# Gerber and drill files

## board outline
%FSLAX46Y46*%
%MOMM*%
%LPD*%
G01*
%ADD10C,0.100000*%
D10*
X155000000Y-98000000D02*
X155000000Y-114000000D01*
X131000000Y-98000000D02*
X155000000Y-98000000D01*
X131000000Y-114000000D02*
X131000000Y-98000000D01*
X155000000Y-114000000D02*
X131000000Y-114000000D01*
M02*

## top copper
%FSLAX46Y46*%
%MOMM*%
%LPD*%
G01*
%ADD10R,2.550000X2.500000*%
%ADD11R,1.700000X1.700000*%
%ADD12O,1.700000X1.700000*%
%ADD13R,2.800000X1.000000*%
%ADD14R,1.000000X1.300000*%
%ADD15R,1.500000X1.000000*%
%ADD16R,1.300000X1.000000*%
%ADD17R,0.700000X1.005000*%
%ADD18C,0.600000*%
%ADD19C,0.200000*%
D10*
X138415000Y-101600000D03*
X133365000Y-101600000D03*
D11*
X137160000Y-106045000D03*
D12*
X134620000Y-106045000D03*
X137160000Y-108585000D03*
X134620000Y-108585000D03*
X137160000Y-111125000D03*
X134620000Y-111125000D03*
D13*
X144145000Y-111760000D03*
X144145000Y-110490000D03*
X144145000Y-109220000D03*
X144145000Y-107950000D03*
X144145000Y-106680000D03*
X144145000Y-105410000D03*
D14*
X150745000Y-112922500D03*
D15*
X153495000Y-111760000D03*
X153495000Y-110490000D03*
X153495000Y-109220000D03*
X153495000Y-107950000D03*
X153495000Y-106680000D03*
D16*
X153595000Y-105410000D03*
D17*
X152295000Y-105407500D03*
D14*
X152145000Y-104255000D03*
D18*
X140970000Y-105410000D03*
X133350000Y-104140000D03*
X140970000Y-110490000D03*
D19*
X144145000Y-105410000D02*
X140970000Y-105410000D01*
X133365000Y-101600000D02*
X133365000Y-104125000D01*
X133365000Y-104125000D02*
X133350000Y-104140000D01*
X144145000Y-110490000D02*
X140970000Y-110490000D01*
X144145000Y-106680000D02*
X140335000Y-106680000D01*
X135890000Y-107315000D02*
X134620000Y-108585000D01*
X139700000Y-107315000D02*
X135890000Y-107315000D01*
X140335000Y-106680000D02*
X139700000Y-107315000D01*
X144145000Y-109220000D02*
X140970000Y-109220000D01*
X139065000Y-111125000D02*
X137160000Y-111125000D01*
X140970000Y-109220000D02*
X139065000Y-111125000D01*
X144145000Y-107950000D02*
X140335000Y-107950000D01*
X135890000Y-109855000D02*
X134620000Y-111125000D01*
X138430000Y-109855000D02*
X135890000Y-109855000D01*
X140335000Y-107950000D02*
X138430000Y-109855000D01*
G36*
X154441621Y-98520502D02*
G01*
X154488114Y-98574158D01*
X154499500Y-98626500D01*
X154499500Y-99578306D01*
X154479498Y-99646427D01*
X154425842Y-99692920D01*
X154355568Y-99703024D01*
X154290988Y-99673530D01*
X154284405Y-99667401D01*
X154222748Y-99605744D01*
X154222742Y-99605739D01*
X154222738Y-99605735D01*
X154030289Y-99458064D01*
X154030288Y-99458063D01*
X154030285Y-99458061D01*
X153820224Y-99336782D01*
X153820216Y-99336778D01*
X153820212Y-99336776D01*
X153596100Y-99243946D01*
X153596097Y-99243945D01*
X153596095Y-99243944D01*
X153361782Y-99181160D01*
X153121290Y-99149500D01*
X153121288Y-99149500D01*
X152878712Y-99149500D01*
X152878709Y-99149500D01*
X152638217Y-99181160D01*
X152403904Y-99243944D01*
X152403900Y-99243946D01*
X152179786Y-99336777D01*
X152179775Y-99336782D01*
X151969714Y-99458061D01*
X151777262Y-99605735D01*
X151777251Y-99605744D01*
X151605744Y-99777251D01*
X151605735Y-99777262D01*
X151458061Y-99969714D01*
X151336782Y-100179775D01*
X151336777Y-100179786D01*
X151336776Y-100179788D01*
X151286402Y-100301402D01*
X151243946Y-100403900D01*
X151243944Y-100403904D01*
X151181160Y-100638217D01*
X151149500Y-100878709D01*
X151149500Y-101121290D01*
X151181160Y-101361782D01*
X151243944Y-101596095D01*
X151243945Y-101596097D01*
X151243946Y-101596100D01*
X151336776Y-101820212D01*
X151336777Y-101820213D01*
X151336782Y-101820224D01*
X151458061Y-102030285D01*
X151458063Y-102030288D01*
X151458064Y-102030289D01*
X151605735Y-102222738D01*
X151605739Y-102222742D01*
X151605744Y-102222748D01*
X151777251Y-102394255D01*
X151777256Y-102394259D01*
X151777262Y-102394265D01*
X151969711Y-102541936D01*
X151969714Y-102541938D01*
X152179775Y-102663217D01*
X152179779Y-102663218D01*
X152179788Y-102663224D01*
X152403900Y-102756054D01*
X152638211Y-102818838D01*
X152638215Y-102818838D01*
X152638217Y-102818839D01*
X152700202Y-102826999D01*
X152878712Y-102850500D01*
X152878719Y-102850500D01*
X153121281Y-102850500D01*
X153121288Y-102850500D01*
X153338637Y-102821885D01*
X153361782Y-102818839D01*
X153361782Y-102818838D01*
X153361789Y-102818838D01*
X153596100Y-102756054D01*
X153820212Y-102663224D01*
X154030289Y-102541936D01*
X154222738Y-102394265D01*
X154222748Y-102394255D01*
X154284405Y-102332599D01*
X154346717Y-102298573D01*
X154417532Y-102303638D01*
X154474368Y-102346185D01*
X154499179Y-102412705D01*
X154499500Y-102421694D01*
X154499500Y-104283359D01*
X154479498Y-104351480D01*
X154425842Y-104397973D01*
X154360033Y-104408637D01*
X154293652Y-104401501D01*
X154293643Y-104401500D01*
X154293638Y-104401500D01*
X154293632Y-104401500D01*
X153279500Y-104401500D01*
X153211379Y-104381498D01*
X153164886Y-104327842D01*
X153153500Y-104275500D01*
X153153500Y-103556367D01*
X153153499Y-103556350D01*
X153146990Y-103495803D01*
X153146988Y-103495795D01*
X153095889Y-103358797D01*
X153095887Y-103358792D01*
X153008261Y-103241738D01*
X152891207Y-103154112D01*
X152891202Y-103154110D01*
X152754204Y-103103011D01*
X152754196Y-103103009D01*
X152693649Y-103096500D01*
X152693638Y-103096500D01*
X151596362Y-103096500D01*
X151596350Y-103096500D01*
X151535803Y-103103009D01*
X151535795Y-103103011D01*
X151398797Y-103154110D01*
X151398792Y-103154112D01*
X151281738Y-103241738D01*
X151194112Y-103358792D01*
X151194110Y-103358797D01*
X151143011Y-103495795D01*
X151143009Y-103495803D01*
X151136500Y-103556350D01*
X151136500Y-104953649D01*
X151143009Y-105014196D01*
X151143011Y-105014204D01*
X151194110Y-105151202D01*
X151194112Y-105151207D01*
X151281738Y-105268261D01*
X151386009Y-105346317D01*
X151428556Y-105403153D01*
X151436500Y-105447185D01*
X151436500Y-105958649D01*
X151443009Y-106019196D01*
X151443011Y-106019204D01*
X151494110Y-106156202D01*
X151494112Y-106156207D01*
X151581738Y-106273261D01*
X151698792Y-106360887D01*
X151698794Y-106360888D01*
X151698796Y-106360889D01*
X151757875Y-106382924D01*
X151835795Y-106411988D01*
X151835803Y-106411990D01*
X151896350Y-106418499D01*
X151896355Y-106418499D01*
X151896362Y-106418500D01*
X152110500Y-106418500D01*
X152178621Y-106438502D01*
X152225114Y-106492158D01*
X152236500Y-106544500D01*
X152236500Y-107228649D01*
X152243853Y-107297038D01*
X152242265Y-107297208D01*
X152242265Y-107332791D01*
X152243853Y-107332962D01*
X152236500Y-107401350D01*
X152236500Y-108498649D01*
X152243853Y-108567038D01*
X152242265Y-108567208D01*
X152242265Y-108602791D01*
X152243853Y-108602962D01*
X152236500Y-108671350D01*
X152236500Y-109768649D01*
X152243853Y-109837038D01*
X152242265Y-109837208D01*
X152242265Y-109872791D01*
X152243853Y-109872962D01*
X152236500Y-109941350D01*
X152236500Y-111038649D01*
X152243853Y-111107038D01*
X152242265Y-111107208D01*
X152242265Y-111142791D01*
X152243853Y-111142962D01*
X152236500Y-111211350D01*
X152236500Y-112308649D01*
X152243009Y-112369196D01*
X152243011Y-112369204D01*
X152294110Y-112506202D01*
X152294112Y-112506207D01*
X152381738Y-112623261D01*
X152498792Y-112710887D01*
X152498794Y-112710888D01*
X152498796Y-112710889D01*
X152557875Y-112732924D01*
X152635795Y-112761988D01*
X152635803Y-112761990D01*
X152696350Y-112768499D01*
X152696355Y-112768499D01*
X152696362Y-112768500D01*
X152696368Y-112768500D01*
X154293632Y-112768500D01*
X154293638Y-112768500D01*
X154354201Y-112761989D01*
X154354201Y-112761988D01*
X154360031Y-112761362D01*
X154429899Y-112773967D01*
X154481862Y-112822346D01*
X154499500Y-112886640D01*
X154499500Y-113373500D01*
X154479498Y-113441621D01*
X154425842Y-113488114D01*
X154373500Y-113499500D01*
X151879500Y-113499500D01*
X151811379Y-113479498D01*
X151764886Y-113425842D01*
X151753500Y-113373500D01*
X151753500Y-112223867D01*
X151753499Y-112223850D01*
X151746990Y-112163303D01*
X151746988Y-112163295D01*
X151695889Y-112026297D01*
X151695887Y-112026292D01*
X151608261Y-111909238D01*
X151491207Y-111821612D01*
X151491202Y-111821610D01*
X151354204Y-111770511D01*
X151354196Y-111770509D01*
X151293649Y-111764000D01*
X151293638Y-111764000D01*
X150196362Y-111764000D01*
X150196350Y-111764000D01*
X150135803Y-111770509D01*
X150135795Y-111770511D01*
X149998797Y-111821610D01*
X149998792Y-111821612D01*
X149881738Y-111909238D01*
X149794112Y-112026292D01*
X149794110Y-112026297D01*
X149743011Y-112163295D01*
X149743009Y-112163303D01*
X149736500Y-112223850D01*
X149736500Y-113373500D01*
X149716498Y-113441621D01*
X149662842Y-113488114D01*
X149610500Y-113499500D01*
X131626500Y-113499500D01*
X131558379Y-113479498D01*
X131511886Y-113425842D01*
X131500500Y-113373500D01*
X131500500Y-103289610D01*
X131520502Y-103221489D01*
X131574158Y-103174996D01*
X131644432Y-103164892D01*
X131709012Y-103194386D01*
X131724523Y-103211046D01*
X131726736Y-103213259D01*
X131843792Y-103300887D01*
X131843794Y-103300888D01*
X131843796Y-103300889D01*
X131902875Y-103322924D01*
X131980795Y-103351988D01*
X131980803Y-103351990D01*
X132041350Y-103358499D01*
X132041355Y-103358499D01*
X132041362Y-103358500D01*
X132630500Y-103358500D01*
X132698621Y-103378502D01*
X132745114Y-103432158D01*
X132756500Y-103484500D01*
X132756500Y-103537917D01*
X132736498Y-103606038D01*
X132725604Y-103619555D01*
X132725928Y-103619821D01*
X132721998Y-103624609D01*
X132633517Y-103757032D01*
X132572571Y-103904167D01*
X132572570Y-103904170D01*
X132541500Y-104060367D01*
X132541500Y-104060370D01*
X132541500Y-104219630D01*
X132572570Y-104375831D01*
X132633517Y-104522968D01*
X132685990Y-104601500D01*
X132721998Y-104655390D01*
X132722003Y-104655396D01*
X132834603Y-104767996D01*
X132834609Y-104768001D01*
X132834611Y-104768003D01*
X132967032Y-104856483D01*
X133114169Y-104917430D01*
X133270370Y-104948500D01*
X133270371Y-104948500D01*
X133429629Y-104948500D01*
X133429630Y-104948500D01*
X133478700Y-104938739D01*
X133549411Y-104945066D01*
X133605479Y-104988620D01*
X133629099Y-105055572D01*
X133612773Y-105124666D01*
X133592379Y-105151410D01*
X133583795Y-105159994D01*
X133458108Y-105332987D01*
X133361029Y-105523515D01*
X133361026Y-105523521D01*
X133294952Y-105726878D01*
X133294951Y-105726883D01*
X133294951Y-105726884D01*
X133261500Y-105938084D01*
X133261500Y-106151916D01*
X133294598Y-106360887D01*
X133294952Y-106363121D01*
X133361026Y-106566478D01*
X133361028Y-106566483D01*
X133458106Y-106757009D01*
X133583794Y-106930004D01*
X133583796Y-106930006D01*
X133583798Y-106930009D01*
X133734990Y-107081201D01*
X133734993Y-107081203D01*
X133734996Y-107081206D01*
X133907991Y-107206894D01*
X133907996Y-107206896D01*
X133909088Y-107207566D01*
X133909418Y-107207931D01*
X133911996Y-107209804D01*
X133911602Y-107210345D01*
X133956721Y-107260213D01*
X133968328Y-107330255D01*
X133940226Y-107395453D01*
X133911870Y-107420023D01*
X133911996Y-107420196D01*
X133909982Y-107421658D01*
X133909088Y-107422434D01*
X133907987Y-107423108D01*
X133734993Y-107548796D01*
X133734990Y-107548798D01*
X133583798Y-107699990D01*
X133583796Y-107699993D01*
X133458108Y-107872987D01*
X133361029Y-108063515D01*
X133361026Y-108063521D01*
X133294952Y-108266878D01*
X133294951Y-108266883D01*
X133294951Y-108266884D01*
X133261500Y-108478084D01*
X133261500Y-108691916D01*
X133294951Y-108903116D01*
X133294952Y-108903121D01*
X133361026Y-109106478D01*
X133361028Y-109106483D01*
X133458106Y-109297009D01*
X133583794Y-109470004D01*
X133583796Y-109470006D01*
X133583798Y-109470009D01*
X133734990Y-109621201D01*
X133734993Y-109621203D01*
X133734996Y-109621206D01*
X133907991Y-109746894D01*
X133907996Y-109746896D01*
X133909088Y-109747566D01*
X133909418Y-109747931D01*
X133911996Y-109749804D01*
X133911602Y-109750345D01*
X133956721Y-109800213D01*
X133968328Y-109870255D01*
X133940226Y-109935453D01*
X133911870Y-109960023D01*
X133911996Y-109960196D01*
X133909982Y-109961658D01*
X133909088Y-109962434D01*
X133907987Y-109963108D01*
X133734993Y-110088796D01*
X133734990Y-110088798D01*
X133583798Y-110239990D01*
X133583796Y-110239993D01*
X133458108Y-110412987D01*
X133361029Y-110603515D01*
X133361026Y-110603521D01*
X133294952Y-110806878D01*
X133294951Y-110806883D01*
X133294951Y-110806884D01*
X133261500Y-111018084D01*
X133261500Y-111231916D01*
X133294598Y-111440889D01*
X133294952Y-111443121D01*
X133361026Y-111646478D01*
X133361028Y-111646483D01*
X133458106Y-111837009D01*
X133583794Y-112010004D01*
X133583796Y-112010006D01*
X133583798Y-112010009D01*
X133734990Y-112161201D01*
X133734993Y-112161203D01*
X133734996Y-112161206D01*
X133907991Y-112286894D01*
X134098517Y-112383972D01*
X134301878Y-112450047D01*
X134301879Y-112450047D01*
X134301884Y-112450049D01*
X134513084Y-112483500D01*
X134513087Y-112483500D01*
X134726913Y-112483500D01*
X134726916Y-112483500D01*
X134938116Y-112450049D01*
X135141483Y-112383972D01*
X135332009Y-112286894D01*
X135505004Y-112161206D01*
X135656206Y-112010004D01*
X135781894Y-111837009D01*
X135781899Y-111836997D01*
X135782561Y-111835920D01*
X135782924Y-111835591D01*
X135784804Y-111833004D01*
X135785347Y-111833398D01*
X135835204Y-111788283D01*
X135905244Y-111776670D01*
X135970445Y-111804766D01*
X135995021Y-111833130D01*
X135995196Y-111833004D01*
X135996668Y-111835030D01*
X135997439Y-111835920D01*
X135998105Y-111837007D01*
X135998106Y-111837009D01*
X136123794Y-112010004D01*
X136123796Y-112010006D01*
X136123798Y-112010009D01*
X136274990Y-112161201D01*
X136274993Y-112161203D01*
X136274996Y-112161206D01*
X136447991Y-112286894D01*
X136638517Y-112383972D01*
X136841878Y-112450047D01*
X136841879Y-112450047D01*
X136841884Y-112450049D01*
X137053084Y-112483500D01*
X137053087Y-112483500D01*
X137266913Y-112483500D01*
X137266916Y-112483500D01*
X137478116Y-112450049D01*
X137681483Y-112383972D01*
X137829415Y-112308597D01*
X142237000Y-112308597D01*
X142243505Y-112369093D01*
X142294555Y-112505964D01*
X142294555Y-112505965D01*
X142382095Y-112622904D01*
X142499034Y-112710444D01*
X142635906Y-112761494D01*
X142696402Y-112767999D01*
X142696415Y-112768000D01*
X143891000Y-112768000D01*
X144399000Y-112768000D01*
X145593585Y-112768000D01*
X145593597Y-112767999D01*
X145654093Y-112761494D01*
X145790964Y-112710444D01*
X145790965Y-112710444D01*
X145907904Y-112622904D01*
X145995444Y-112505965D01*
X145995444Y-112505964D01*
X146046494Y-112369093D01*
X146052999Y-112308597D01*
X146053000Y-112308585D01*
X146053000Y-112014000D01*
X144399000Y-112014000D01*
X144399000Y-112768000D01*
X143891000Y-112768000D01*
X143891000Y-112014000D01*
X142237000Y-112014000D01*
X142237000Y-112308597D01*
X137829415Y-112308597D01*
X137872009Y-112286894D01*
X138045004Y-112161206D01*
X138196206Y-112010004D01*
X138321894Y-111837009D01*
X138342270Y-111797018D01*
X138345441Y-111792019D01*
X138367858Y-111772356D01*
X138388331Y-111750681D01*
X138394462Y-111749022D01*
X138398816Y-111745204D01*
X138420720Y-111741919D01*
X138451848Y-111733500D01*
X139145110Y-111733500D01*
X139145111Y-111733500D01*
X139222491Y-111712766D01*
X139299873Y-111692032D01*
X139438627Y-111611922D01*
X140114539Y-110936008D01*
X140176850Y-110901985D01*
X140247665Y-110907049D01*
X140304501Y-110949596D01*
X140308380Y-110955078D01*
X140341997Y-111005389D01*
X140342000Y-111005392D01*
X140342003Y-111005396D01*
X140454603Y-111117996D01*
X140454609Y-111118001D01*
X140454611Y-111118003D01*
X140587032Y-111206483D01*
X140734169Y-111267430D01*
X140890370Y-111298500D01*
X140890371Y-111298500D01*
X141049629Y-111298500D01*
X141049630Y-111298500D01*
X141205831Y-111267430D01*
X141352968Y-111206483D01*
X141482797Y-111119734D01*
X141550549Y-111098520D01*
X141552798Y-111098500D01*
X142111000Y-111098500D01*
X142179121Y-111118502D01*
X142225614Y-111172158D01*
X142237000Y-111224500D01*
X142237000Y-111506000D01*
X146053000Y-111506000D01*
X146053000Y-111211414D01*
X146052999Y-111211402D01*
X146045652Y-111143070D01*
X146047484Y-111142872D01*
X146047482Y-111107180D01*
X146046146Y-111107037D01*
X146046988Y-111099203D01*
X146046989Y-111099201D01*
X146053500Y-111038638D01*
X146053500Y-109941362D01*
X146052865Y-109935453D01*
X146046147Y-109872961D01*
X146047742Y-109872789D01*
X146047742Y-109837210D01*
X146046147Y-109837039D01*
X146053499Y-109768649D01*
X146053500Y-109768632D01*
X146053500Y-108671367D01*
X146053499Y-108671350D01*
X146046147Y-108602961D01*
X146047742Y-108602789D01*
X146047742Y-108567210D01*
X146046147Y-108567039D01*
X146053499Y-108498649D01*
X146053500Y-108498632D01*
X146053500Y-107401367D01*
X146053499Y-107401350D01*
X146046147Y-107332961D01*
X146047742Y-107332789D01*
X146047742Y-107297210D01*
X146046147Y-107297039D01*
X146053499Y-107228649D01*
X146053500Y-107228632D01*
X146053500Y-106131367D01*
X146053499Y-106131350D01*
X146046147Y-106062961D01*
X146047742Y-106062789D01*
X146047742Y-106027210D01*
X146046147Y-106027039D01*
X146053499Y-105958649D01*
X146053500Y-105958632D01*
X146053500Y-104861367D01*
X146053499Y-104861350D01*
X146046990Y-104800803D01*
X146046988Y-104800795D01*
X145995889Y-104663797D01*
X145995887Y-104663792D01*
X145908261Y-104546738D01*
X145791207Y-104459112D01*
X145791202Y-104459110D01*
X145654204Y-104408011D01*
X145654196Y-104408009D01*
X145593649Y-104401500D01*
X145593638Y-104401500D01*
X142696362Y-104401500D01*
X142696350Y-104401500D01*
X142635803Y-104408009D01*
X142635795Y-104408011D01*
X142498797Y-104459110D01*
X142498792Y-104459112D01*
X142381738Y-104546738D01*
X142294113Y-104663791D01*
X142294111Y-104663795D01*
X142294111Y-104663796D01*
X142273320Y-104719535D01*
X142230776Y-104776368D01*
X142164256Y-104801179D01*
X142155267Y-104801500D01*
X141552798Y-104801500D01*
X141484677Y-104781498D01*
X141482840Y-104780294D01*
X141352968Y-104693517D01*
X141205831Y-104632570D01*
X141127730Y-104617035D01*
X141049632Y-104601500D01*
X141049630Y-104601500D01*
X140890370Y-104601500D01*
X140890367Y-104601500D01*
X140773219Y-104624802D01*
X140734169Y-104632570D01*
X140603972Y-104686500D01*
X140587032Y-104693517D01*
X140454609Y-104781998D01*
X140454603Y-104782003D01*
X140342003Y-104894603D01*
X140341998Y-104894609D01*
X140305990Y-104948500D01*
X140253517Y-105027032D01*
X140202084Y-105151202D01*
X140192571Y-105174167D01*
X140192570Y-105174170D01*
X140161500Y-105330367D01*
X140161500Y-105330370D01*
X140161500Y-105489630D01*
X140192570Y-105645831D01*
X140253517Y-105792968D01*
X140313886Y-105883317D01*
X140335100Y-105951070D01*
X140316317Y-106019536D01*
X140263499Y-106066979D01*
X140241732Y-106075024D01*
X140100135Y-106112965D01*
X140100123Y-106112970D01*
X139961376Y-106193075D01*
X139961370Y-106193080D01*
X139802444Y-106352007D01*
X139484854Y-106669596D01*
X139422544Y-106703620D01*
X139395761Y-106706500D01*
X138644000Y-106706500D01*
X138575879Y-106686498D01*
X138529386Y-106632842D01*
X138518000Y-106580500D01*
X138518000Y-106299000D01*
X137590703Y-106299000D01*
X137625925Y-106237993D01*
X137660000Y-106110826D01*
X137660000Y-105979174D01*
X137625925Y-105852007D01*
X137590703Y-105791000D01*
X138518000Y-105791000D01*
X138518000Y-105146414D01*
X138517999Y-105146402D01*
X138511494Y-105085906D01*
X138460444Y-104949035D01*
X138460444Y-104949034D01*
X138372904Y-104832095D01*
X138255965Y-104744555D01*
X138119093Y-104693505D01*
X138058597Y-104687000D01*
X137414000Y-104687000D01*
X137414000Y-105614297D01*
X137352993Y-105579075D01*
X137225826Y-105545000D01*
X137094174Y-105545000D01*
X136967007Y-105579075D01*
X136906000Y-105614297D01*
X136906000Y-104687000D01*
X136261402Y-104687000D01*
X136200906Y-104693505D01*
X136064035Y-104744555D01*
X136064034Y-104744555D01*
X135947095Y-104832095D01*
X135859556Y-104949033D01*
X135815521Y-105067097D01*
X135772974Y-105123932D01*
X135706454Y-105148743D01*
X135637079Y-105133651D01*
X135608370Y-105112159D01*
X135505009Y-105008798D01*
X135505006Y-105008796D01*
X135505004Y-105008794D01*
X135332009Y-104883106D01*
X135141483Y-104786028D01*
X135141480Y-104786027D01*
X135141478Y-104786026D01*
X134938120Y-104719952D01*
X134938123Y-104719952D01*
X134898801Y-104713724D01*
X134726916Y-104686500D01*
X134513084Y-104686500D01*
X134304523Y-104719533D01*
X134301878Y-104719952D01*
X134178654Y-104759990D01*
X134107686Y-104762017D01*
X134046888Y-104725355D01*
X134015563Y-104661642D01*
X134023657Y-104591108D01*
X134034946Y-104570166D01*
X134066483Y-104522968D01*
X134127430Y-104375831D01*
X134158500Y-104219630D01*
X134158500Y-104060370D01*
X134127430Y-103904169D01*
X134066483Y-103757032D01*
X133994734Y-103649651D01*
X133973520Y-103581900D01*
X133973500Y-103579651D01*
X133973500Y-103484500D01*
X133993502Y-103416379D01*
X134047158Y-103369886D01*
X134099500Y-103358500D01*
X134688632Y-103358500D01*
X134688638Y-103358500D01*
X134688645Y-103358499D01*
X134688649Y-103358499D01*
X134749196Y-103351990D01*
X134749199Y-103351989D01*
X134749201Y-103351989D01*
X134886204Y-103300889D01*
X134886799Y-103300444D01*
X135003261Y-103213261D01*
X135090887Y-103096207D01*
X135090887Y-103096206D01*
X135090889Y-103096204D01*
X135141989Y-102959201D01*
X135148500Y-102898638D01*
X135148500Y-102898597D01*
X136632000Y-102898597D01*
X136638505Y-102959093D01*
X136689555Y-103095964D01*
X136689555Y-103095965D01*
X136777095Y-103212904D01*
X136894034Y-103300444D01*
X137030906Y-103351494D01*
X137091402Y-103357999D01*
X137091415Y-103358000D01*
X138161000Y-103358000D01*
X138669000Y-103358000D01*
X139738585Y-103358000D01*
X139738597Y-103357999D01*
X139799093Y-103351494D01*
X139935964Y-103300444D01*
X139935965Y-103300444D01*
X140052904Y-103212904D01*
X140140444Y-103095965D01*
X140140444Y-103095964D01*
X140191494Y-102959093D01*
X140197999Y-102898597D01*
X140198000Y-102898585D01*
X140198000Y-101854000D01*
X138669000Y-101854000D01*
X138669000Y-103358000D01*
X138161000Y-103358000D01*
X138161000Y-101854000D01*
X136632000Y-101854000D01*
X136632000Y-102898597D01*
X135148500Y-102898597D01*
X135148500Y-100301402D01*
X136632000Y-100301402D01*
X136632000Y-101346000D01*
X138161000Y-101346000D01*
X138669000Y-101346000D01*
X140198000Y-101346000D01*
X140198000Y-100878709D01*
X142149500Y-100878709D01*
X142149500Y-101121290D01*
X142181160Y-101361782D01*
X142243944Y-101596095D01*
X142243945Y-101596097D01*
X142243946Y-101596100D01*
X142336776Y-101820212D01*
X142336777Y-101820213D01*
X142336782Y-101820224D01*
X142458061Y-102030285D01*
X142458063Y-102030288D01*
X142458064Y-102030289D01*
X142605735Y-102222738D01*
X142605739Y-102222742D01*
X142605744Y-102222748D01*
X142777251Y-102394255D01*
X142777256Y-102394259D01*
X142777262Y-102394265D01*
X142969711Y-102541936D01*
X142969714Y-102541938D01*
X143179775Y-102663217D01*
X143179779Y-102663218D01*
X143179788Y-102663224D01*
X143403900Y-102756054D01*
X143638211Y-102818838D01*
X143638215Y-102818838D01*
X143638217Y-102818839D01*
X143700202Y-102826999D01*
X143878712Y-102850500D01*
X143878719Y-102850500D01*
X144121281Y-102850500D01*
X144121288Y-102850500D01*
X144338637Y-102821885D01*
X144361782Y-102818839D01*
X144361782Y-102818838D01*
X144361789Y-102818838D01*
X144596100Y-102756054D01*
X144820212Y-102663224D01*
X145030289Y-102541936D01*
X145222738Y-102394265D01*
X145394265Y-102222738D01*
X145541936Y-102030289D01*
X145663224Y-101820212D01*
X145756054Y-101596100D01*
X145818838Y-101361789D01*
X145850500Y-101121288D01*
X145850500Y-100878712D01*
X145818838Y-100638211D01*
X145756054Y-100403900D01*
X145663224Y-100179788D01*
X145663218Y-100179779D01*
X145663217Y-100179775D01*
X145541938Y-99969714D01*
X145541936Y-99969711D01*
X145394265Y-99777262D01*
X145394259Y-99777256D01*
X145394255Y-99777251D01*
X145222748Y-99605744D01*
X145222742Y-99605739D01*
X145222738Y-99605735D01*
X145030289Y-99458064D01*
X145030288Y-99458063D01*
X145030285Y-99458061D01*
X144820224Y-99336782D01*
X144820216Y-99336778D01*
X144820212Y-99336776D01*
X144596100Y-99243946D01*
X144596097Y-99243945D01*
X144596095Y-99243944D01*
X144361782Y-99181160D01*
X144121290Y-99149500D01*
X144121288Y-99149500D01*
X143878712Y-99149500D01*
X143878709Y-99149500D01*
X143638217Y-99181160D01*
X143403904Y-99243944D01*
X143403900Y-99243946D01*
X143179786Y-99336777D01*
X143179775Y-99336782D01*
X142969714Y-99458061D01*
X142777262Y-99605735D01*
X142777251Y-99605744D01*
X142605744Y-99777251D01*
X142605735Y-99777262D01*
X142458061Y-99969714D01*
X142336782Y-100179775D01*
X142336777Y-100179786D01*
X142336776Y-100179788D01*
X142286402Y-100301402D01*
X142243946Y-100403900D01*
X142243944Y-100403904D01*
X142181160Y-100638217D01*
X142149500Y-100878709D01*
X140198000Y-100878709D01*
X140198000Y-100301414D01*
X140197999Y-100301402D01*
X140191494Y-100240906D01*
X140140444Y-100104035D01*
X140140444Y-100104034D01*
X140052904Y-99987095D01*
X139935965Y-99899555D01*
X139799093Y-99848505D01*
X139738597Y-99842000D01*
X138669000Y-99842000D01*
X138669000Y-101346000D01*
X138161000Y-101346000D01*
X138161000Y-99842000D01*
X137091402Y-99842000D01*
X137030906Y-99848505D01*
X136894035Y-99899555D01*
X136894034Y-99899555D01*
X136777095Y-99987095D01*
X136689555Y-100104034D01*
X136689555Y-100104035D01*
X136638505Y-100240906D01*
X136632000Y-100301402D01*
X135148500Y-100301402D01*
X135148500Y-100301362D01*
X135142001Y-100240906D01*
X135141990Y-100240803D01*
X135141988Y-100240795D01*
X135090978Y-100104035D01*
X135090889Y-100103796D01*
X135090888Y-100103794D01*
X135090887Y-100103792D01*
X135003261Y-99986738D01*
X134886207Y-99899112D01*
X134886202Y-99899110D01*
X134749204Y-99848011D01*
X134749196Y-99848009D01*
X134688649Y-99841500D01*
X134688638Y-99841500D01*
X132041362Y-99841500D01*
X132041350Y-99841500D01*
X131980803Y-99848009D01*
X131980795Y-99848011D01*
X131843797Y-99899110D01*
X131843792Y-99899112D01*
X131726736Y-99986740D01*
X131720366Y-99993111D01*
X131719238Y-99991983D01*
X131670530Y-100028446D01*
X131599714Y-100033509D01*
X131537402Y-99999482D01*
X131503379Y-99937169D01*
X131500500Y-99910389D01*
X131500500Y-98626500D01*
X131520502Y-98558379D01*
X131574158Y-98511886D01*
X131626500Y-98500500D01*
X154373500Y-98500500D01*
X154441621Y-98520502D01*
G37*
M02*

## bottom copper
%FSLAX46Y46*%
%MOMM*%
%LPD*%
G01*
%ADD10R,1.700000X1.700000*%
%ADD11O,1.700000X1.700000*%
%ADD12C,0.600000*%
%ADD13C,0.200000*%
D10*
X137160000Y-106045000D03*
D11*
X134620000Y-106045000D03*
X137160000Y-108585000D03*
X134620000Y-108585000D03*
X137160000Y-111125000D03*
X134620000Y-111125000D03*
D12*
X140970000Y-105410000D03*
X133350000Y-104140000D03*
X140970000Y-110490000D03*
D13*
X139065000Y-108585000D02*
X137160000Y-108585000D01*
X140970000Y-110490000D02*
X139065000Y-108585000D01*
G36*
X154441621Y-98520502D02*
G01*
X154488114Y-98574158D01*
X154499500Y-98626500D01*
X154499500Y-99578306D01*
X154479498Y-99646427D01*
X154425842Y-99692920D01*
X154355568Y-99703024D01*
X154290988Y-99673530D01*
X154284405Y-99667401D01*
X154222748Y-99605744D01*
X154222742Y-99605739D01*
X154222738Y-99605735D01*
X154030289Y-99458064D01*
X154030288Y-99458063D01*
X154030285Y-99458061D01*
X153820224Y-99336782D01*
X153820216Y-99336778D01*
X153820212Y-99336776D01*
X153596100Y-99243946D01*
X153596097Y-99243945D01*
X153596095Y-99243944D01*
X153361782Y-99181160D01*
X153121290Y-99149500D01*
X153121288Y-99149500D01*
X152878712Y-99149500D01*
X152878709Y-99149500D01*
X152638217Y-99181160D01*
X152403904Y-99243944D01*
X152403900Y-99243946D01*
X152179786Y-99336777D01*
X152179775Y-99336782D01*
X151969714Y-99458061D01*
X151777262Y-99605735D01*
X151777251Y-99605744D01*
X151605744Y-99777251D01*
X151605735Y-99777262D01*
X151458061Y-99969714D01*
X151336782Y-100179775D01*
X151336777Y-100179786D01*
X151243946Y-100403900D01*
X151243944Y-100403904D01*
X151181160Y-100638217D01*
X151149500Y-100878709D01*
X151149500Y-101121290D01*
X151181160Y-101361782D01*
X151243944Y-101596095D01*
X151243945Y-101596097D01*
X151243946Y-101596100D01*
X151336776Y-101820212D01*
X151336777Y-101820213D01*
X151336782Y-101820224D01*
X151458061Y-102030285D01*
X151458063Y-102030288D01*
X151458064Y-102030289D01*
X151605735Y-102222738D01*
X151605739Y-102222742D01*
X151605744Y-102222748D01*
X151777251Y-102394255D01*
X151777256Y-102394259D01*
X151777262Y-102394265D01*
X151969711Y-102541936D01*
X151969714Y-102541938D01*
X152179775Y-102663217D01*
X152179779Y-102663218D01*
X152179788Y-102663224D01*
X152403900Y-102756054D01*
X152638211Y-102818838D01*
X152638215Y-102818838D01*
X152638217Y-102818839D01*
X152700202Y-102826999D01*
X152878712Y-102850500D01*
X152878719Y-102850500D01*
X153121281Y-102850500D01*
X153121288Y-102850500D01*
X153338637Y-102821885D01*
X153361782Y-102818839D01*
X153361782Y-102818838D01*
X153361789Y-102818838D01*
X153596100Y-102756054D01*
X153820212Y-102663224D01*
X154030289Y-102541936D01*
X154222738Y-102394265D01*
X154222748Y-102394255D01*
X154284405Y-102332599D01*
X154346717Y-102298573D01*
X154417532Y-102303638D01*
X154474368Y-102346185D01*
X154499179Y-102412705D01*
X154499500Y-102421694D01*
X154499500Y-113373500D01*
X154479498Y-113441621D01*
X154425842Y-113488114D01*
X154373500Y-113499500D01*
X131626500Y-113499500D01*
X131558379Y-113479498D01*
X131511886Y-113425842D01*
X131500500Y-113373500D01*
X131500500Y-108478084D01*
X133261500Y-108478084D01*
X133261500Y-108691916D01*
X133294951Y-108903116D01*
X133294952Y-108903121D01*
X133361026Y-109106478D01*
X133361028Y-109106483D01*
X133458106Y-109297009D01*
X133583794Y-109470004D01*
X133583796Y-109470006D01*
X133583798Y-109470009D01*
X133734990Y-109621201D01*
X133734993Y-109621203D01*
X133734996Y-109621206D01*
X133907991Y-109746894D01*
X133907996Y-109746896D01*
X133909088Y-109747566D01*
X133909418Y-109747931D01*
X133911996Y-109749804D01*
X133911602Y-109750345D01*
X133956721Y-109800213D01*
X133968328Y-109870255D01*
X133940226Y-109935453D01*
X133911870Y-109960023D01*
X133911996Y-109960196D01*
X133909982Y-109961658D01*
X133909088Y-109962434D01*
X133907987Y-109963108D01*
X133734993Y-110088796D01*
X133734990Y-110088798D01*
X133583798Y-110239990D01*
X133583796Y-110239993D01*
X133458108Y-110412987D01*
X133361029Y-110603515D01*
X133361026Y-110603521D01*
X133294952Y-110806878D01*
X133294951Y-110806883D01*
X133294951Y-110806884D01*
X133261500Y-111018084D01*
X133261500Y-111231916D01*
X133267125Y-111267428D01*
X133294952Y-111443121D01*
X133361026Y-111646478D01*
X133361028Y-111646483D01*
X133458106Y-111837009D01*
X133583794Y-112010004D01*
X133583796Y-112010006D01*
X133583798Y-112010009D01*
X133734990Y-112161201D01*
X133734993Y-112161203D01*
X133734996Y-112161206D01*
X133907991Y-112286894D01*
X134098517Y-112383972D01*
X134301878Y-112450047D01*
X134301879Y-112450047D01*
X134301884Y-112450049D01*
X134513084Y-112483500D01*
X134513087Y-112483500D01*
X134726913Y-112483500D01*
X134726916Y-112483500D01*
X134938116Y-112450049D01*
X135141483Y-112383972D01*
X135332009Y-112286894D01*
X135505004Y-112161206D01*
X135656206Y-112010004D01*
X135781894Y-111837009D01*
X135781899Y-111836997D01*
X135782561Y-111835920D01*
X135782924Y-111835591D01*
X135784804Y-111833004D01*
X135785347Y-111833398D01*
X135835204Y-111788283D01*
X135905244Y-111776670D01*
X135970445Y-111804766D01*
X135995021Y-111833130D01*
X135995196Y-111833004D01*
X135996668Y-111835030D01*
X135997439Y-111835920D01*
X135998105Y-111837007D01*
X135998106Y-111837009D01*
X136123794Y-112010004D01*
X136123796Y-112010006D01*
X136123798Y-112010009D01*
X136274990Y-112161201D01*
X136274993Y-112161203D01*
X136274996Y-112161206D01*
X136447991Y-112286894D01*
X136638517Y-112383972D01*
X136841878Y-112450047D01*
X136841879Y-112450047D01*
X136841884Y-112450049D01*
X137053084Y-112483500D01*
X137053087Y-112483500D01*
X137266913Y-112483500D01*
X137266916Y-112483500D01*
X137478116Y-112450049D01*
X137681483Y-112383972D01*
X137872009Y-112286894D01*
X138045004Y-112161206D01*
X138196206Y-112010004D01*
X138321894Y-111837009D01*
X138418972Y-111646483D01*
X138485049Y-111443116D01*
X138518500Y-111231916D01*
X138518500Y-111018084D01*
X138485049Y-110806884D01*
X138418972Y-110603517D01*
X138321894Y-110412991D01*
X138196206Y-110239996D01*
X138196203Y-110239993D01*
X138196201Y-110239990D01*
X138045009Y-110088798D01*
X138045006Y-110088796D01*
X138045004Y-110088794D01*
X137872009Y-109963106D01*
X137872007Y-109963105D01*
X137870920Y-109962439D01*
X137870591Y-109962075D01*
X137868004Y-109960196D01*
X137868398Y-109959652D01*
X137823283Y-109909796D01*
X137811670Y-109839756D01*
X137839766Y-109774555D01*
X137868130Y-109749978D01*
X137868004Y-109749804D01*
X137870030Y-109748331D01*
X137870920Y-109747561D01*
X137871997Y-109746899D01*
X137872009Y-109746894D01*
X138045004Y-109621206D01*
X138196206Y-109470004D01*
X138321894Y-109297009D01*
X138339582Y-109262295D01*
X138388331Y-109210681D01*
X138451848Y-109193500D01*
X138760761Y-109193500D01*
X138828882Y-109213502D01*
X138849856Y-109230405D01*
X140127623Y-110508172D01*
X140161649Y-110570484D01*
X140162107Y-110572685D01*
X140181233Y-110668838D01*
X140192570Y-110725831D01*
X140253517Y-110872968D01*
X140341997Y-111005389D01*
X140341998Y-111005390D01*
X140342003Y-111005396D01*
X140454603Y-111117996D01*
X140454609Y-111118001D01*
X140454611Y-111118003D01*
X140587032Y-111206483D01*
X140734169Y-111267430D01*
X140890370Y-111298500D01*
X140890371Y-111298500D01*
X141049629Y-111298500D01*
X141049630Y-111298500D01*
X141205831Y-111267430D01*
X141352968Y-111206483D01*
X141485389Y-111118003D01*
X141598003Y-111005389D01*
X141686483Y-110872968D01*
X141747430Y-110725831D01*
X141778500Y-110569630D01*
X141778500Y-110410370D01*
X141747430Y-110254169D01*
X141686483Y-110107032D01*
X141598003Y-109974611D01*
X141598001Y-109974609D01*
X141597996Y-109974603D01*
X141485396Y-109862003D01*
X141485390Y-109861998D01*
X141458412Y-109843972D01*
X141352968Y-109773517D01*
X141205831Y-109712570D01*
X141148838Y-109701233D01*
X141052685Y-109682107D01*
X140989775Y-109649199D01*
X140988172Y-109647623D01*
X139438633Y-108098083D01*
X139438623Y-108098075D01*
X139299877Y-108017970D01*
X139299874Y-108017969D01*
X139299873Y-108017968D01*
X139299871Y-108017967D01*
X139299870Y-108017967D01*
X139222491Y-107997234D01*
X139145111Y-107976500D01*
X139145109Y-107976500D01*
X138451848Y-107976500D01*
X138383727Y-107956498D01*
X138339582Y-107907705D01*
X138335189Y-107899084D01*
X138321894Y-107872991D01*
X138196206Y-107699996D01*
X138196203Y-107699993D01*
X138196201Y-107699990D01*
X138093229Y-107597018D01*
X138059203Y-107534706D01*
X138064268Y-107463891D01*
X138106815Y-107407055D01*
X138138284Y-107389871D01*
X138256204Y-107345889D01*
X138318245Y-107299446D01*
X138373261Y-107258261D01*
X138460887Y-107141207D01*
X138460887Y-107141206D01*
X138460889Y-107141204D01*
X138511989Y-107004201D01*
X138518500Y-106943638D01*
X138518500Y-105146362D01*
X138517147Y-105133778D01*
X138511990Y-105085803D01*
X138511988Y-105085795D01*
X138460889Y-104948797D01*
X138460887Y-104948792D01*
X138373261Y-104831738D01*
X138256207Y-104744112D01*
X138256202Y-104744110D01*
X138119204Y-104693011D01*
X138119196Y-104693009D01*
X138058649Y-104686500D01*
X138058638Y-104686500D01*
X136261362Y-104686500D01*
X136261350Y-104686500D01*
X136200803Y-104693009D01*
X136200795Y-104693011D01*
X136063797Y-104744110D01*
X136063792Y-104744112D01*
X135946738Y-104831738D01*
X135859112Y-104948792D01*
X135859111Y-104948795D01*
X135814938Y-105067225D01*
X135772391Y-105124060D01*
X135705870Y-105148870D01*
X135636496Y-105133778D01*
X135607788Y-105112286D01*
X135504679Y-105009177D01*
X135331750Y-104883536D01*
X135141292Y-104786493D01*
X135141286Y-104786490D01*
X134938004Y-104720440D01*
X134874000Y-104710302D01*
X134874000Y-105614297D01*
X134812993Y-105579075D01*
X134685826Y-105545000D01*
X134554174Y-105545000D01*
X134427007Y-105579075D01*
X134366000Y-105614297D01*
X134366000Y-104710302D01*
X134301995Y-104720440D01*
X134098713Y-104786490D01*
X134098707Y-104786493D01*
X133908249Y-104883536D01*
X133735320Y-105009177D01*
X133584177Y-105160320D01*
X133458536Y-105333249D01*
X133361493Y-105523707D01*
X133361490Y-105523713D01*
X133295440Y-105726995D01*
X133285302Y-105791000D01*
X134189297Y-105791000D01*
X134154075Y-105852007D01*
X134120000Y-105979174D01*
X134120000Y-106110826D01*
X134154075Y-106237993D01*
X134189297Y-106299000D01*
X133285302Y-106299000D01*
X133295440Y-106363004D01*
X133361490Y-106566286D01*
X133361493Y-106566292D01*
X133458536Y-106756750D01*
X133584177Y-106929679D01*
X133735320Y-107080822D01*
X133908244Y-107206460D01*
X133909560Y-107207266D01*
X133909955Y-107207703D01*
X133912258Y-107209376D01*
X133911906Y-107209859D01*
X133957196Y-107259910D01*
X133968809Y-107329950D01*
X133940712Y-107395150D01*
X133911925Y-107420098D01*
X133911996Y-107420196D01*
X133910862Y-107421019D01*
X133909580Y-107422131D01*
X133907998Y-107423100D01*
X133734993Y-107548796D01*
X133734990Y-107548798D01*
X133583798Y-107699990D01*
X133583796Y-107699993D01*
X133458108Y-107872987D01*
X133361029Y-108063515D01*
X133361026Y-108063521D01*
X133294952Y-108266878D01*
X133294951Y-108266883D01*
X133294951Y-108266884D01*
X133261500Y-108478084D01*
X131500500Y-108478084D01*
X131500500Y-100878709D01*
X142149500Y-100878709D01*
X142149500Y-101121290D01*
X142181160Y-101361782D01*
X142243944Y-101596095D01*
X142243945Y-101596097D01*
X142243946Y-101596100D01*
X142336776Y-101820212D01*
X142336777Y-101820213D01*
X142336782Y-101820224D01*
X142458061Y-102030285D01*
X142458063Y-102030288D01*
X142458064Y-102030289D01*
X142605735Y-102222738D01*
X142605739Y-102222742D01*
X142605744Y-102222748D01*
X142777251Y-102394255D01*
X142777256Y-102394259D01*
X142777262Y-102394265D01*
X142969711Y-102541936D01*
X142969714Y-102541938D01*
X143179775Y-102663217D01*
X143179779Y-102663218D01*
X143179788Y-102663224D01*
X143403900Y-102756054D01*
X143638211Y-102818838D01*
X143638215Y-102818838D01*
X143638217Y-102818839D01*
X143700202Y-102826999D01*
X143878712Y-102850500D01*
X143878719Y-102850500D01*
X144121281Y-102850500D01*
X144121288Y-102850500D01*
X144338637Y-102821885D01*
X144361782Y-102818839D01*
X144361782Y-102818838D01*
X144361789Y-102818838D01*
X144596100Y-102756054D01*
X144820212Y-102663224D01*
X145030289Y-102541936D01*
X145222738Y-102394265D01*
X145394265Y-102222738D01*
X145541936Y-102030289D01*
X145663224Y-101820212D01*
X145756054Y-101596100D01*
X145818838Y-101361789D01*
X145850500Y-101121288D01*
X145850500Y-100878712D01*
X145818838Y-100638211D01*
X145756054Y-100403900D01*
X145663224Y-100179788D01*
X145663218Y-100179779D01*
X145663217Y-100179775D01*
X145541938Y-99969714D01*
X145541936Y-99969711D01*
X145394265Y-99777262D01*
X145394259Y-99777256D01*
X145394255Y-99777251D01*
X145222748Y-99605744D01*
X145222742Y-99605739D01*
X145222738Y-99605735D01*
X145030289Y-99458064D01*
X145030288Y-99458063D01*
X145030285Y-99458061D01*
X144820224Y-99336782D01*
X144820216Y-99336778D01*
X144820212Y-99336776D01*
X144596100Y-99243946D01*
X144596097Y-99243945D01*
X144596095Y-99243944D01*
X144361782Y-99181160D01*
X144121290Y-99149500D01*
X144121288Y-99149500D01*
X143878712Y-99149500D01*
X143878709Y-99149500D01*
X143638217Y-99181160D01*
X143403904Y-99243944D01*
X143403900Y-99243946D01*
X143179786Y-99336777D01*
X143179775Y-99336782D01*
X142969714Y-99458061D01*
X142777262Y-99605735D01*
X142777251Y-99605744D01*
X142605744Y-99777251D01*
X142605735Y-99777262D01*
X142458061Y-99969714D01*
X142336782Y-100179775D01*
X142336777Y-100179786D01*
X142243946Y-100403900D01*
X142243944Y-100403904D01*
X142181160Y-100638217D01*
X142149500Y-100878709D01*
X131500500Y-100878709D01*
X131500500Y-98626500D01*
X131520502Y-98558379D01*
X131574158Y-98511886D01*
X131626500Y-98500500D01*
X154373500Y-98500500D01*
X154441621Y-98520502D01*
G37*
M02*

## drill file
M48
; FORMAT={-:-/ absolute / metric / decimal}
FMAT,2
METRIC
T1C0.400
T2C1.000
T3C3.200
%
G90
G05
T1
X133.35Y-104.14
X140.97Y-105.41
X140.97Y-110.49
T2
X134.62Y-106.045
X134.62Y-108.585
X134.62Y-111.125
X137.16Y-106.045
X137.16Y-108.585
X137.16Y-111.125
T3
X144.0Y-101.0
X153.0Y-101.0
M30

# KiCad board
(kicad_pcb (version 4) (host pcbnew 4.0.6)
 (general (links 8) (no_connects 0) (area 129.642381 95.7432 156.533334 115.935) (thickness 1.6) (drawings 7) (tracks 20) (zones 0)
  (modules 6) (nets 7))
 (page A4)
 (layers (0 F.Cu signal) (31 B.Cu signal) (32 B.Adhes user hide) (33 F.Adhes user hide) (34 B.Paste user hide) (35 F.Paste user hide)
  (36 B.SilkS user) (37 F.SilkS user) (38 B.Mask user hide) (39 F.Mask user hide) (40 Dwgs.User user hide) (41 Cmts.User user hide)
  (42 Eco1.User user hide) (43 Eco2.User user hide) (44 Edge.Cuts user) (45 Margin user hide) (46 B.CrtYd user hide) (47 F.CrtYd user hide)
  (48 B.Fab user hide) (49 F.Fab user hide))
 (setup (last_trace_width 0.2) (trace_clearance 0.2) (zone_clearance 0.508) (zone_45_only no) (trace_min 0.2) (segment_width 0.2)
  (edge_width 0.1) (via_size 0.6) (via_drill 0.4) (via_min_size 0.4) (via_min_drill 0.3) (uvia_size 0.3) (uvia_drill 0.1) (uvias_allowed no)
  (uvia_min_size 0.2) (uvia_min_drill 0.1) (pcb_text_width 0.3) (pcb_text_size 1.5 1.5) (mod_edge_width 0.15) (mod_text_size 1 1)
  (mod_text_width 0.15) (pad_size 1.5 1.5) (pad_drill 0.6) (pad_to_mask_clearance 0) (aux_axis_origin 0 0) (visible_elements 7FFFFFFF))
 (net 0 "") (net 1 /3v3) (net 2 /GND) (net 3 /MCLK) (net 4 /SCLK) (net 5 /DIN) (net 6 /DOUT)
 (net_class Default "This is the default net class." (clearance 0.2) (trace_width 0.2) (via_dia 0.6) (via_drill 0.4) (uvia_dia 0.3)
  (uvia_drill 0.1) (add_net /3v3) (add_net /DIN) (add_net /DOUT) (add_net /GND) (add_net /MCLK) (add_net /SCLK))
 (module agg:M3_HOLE (layer F.Cu) (at 144 101)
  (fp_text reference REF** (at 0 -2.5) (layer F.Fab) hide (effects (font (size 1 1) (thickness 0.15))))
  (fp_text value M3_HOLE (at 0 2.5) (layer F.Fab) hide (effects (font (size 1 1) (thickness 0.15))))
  (pad "" np_thru_hole circle (at 0 0) (size 3.2 3.2) (drill 3.2) (layers *.Cu F.Mask)))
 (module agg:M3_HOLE (layer F.Cu) (at 153 101)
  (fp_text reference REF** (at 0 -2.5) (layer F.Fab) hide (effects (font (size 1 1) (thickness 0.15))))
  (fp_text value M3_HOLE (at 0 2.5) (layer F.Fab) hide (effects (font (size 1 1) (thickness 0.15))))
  (pad "" np_thru_hole circle (at 0 0) (size 3.2 3.2) (drill 3.2) (layers *.Cu F.Mask)))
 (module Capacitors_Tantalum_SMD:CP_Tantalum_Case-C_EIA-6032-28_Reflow (layer F.Cu) (at 135.89 101.6 180)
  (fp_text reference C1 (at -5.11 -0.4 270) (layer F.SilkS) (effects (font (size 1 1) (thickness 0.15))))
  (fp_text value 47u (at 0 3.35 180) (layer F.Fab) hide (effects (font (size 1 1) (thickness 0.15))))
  (pad 1 smd rect (at -2.525 0 180) (size 2.55 2.5) (layers F.Cu F.Paste F.Mask) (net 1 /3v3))
  (pad 2 smd rect (at 2.525 0 180) (size 2.55 2.5) (layers F.Cu F.Paste F.Mask) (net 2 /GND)))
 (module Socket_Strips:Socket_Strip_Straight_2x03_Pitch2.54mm (layer F.Cu) (at 137.16 106.045)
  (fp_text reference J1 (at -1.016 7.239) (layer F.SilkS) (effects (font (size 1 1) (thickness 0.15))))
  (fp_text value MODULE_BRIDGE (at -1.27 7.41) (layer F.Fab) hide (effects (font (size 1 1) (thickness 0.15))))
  (pad 1 thru_hole rect (at 0 0) (size 1.7 1.7) (drill 1) (layers *.Cu *.Mask) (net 1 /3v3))
  (pad 2 thru_hole oval (at -2.54 0) (size 1.7 1.7) (drill 1) (layers *.Cu *.Mask) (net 2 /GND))
  (pad 3 thru_hole oval (at 0 2.54) (size 1.7 1.7) (drill 1) (layers *.Cu *.Mask) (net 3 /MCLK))
  (pad 4 thru_hole oval (at -2.54 2.54) (size 1.7 1.7) (drill 1) (layers *.Cu *.Mask) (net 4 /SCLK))
  (pad 5 thru_hole oval (at 0 5.08) (size 1.7 1.7) (drill 1) (layers *.Cu *.Mask) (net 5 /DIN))
  (pad 6 thru_hole oval (at -2.54 5.08) (size 1.7 1.7) (drill 1) (layers *.Cu *.Mask) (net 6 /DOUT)))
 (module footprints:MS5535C (layer F.Cu) (at 144.145 111.76 180)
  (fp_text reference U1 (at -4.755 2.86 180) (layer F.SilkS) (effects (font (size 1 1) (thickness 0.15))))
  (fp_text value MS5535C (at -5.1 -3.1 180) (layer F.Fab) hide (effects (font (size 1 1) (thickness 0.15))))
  (pad 6 smd rect (at 0 0 180) (size 2.8 1) (layers F.Cu F.Paste F.Mask) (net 1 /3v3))
  (pad 5 smd rect (at 0 1.27 180) (size 2.8 1) (layers F.Cu F.Paste F.Mask) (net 3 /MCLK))
  (pad 4 smd rect (at 0 2.54 180) (size 2.8 1) (layers F.Cu F.Paste F.Mask) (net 5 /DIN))
  (pad 3 smd rect (at 0 3.81 180) (size 2.8 1) (layers F.Cu F.Paste F.Mask) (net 6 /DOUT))
  (pad 2 smd rect (at 0 5.08 180) (size 2.8 1) (layers F.Cu F.Paste F.Mask) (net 4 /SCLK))
  (pad 1 smd rect (at 0 6.35 180) (size 2.8 1) (layers F.Cu F.Paste F.Mask) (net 2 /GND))
  (pad 7 smd rect (at -6.6 -1.1625 180) (size 1 1.3) (layers F.Cu F.Paste F.Mask))
  (pad 8 smd rect (at -9.35 0 180) (size 1.5 1) (layers F.Cu F.Paste F.Mask))
  (pad 9 smd rect (at -9.35 1.27 180) (size 1.5 1) (layers F.Cu F.Paste F.Mask))
  (pad 10 smd rect (at -9.35 2.54 180) (size 1.5 1) (layers F.Cu F.Paste F.Mask))
  (pad 11 smd rect (at -9.35 3.81 180) (size 1.5 1) (layers F.Cu F.Paste F.Mask))
  (pad 12 smd rect (at -9.35 5.08 180) (size 1.5 1) (layers F.Cu F.Paste F.Mask))
  (pad 13 smd rect (at -9.45 6.35 180) (size 1.3 1) (layers F.Cu F.Paste F.Mask))
  (pad 14 smd rect (at -8.15 6.3525 180) (size 0.7 1.005) (layers F.Cu F.Paste F.Mask))
  (pad 14 smd rect (at -8 7.505 180) (size 1 1.3) (layers F.Cu F.Paste F.Mask)))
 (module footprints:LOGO (layer F.Cu) (at 148.5 99.7)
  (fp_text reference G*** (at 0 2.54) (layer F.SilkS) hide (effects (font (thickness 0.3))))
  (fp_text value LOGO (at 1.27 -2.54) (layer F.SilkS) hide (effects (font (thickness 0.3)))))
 (gr_line (start 155 98) (end 155 114) (layer Edge.Cuts) (width 0.1))
 (gr_line (start 131 98) (end 155 98) (layer Edge.Cuts) (width 0.1))
 (gr_line (start 131 114) (end 131 98) (layer Edge.Cuts) (width 0.1))
 (gr_line (start 155 114) (end 131 114) (layer Edge.Cuts) (width 0.1))
 (segment (start 144.145 105.41) (end 140.97 105.41) (width 0.2) (layer F.Cu) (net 2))
 (via (at 140.97 105.41) (size 0.6) (drill 0.4) (layers F.Cu B.Cu) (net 2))
 (segment (start 133.365 101.6) (end 133.365 104.125) (width 0.2) (layer F.Cu) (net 2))
 (via (at 133.35 104.14) (size 0.6) (drill 0.4) (layers F.Cu B.Cu) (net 2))
 (segment (start 133.365 104.125) (end 133.35 104.14) (width 0.2) (layer F.Cu) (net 2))
 (segment (start 139.065 108.585) (end 137.16 108.585) (width 0.2) (layer B.Cu) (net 3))
 (segment (start 144.145 110.49) (end 140.97 110.49) (width 0.2) (layer F.Cu) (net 3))
 (segment (start 140.97 110.49) (end 139.065 108.585) (width 0.2) (layer B.Cu) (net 3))
 (via (at 140.97 110.49) (size 0.6) (drill 0.4) (layers F.Cu B.Cu) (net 3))
 (segment (start 144.145 106.68) (end 140.335 106.68) (width 0.2) (layer F.Cu) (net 4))
 (segment (start 135.89 107.315) (end 134.62 108.585) (width 0.2) (layer F.Cu) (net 4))
 (segment (start 139.7 107.315) (end 135.89 107.315) (width 0.2) (layer F.Cu) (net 4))
 (segment (start 140.335 106.68) (end 139.7 107.315) (width 0.2) (layer F.Cu) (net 4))
 (segment (start 144.145 109.22) (end 140.97 109.22) (width 0.2) (layer F.Cu) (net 5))
 (segment (start 139.065 111.125) (end 137.16 111.125) (width 0.2) (layer F.Cu) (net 5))
 (segment (start 140.97 109.22) (end 139.065 111.125) (width 0.2) (layer F.Cu) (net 5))
 (segment (start 144.145 107.95) (end 140.335 107.95) (width 0.2) (layer F.Cu) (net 6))
 (segment (start 135.89 109.855) (end 134.62 111.125) (width 0.2) (layer F.Cu) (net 6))
 (segment (start 138.43 109.855) (end 135.89 109.855) (width 0.2) (layer F.Cu) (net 6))
 (segment (start 140.335 107.95) (end 138.43 109.855) (width 0.2) (layer F.Cu) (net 6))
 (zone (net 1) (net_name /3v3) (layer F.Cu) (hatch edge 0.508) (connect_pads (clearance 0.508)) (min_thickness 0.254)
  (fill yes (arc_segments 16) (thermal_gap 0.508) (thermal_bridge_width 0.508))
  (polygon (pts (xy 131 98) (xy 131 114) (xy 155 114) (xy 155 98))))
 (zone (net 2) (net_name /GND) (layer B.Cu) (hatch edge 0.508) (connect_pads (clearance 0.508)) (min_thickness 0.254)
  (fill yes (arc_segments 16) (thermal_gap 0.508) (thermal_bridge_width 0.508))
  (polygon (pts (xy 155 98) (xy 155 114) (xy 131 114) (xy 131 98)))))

